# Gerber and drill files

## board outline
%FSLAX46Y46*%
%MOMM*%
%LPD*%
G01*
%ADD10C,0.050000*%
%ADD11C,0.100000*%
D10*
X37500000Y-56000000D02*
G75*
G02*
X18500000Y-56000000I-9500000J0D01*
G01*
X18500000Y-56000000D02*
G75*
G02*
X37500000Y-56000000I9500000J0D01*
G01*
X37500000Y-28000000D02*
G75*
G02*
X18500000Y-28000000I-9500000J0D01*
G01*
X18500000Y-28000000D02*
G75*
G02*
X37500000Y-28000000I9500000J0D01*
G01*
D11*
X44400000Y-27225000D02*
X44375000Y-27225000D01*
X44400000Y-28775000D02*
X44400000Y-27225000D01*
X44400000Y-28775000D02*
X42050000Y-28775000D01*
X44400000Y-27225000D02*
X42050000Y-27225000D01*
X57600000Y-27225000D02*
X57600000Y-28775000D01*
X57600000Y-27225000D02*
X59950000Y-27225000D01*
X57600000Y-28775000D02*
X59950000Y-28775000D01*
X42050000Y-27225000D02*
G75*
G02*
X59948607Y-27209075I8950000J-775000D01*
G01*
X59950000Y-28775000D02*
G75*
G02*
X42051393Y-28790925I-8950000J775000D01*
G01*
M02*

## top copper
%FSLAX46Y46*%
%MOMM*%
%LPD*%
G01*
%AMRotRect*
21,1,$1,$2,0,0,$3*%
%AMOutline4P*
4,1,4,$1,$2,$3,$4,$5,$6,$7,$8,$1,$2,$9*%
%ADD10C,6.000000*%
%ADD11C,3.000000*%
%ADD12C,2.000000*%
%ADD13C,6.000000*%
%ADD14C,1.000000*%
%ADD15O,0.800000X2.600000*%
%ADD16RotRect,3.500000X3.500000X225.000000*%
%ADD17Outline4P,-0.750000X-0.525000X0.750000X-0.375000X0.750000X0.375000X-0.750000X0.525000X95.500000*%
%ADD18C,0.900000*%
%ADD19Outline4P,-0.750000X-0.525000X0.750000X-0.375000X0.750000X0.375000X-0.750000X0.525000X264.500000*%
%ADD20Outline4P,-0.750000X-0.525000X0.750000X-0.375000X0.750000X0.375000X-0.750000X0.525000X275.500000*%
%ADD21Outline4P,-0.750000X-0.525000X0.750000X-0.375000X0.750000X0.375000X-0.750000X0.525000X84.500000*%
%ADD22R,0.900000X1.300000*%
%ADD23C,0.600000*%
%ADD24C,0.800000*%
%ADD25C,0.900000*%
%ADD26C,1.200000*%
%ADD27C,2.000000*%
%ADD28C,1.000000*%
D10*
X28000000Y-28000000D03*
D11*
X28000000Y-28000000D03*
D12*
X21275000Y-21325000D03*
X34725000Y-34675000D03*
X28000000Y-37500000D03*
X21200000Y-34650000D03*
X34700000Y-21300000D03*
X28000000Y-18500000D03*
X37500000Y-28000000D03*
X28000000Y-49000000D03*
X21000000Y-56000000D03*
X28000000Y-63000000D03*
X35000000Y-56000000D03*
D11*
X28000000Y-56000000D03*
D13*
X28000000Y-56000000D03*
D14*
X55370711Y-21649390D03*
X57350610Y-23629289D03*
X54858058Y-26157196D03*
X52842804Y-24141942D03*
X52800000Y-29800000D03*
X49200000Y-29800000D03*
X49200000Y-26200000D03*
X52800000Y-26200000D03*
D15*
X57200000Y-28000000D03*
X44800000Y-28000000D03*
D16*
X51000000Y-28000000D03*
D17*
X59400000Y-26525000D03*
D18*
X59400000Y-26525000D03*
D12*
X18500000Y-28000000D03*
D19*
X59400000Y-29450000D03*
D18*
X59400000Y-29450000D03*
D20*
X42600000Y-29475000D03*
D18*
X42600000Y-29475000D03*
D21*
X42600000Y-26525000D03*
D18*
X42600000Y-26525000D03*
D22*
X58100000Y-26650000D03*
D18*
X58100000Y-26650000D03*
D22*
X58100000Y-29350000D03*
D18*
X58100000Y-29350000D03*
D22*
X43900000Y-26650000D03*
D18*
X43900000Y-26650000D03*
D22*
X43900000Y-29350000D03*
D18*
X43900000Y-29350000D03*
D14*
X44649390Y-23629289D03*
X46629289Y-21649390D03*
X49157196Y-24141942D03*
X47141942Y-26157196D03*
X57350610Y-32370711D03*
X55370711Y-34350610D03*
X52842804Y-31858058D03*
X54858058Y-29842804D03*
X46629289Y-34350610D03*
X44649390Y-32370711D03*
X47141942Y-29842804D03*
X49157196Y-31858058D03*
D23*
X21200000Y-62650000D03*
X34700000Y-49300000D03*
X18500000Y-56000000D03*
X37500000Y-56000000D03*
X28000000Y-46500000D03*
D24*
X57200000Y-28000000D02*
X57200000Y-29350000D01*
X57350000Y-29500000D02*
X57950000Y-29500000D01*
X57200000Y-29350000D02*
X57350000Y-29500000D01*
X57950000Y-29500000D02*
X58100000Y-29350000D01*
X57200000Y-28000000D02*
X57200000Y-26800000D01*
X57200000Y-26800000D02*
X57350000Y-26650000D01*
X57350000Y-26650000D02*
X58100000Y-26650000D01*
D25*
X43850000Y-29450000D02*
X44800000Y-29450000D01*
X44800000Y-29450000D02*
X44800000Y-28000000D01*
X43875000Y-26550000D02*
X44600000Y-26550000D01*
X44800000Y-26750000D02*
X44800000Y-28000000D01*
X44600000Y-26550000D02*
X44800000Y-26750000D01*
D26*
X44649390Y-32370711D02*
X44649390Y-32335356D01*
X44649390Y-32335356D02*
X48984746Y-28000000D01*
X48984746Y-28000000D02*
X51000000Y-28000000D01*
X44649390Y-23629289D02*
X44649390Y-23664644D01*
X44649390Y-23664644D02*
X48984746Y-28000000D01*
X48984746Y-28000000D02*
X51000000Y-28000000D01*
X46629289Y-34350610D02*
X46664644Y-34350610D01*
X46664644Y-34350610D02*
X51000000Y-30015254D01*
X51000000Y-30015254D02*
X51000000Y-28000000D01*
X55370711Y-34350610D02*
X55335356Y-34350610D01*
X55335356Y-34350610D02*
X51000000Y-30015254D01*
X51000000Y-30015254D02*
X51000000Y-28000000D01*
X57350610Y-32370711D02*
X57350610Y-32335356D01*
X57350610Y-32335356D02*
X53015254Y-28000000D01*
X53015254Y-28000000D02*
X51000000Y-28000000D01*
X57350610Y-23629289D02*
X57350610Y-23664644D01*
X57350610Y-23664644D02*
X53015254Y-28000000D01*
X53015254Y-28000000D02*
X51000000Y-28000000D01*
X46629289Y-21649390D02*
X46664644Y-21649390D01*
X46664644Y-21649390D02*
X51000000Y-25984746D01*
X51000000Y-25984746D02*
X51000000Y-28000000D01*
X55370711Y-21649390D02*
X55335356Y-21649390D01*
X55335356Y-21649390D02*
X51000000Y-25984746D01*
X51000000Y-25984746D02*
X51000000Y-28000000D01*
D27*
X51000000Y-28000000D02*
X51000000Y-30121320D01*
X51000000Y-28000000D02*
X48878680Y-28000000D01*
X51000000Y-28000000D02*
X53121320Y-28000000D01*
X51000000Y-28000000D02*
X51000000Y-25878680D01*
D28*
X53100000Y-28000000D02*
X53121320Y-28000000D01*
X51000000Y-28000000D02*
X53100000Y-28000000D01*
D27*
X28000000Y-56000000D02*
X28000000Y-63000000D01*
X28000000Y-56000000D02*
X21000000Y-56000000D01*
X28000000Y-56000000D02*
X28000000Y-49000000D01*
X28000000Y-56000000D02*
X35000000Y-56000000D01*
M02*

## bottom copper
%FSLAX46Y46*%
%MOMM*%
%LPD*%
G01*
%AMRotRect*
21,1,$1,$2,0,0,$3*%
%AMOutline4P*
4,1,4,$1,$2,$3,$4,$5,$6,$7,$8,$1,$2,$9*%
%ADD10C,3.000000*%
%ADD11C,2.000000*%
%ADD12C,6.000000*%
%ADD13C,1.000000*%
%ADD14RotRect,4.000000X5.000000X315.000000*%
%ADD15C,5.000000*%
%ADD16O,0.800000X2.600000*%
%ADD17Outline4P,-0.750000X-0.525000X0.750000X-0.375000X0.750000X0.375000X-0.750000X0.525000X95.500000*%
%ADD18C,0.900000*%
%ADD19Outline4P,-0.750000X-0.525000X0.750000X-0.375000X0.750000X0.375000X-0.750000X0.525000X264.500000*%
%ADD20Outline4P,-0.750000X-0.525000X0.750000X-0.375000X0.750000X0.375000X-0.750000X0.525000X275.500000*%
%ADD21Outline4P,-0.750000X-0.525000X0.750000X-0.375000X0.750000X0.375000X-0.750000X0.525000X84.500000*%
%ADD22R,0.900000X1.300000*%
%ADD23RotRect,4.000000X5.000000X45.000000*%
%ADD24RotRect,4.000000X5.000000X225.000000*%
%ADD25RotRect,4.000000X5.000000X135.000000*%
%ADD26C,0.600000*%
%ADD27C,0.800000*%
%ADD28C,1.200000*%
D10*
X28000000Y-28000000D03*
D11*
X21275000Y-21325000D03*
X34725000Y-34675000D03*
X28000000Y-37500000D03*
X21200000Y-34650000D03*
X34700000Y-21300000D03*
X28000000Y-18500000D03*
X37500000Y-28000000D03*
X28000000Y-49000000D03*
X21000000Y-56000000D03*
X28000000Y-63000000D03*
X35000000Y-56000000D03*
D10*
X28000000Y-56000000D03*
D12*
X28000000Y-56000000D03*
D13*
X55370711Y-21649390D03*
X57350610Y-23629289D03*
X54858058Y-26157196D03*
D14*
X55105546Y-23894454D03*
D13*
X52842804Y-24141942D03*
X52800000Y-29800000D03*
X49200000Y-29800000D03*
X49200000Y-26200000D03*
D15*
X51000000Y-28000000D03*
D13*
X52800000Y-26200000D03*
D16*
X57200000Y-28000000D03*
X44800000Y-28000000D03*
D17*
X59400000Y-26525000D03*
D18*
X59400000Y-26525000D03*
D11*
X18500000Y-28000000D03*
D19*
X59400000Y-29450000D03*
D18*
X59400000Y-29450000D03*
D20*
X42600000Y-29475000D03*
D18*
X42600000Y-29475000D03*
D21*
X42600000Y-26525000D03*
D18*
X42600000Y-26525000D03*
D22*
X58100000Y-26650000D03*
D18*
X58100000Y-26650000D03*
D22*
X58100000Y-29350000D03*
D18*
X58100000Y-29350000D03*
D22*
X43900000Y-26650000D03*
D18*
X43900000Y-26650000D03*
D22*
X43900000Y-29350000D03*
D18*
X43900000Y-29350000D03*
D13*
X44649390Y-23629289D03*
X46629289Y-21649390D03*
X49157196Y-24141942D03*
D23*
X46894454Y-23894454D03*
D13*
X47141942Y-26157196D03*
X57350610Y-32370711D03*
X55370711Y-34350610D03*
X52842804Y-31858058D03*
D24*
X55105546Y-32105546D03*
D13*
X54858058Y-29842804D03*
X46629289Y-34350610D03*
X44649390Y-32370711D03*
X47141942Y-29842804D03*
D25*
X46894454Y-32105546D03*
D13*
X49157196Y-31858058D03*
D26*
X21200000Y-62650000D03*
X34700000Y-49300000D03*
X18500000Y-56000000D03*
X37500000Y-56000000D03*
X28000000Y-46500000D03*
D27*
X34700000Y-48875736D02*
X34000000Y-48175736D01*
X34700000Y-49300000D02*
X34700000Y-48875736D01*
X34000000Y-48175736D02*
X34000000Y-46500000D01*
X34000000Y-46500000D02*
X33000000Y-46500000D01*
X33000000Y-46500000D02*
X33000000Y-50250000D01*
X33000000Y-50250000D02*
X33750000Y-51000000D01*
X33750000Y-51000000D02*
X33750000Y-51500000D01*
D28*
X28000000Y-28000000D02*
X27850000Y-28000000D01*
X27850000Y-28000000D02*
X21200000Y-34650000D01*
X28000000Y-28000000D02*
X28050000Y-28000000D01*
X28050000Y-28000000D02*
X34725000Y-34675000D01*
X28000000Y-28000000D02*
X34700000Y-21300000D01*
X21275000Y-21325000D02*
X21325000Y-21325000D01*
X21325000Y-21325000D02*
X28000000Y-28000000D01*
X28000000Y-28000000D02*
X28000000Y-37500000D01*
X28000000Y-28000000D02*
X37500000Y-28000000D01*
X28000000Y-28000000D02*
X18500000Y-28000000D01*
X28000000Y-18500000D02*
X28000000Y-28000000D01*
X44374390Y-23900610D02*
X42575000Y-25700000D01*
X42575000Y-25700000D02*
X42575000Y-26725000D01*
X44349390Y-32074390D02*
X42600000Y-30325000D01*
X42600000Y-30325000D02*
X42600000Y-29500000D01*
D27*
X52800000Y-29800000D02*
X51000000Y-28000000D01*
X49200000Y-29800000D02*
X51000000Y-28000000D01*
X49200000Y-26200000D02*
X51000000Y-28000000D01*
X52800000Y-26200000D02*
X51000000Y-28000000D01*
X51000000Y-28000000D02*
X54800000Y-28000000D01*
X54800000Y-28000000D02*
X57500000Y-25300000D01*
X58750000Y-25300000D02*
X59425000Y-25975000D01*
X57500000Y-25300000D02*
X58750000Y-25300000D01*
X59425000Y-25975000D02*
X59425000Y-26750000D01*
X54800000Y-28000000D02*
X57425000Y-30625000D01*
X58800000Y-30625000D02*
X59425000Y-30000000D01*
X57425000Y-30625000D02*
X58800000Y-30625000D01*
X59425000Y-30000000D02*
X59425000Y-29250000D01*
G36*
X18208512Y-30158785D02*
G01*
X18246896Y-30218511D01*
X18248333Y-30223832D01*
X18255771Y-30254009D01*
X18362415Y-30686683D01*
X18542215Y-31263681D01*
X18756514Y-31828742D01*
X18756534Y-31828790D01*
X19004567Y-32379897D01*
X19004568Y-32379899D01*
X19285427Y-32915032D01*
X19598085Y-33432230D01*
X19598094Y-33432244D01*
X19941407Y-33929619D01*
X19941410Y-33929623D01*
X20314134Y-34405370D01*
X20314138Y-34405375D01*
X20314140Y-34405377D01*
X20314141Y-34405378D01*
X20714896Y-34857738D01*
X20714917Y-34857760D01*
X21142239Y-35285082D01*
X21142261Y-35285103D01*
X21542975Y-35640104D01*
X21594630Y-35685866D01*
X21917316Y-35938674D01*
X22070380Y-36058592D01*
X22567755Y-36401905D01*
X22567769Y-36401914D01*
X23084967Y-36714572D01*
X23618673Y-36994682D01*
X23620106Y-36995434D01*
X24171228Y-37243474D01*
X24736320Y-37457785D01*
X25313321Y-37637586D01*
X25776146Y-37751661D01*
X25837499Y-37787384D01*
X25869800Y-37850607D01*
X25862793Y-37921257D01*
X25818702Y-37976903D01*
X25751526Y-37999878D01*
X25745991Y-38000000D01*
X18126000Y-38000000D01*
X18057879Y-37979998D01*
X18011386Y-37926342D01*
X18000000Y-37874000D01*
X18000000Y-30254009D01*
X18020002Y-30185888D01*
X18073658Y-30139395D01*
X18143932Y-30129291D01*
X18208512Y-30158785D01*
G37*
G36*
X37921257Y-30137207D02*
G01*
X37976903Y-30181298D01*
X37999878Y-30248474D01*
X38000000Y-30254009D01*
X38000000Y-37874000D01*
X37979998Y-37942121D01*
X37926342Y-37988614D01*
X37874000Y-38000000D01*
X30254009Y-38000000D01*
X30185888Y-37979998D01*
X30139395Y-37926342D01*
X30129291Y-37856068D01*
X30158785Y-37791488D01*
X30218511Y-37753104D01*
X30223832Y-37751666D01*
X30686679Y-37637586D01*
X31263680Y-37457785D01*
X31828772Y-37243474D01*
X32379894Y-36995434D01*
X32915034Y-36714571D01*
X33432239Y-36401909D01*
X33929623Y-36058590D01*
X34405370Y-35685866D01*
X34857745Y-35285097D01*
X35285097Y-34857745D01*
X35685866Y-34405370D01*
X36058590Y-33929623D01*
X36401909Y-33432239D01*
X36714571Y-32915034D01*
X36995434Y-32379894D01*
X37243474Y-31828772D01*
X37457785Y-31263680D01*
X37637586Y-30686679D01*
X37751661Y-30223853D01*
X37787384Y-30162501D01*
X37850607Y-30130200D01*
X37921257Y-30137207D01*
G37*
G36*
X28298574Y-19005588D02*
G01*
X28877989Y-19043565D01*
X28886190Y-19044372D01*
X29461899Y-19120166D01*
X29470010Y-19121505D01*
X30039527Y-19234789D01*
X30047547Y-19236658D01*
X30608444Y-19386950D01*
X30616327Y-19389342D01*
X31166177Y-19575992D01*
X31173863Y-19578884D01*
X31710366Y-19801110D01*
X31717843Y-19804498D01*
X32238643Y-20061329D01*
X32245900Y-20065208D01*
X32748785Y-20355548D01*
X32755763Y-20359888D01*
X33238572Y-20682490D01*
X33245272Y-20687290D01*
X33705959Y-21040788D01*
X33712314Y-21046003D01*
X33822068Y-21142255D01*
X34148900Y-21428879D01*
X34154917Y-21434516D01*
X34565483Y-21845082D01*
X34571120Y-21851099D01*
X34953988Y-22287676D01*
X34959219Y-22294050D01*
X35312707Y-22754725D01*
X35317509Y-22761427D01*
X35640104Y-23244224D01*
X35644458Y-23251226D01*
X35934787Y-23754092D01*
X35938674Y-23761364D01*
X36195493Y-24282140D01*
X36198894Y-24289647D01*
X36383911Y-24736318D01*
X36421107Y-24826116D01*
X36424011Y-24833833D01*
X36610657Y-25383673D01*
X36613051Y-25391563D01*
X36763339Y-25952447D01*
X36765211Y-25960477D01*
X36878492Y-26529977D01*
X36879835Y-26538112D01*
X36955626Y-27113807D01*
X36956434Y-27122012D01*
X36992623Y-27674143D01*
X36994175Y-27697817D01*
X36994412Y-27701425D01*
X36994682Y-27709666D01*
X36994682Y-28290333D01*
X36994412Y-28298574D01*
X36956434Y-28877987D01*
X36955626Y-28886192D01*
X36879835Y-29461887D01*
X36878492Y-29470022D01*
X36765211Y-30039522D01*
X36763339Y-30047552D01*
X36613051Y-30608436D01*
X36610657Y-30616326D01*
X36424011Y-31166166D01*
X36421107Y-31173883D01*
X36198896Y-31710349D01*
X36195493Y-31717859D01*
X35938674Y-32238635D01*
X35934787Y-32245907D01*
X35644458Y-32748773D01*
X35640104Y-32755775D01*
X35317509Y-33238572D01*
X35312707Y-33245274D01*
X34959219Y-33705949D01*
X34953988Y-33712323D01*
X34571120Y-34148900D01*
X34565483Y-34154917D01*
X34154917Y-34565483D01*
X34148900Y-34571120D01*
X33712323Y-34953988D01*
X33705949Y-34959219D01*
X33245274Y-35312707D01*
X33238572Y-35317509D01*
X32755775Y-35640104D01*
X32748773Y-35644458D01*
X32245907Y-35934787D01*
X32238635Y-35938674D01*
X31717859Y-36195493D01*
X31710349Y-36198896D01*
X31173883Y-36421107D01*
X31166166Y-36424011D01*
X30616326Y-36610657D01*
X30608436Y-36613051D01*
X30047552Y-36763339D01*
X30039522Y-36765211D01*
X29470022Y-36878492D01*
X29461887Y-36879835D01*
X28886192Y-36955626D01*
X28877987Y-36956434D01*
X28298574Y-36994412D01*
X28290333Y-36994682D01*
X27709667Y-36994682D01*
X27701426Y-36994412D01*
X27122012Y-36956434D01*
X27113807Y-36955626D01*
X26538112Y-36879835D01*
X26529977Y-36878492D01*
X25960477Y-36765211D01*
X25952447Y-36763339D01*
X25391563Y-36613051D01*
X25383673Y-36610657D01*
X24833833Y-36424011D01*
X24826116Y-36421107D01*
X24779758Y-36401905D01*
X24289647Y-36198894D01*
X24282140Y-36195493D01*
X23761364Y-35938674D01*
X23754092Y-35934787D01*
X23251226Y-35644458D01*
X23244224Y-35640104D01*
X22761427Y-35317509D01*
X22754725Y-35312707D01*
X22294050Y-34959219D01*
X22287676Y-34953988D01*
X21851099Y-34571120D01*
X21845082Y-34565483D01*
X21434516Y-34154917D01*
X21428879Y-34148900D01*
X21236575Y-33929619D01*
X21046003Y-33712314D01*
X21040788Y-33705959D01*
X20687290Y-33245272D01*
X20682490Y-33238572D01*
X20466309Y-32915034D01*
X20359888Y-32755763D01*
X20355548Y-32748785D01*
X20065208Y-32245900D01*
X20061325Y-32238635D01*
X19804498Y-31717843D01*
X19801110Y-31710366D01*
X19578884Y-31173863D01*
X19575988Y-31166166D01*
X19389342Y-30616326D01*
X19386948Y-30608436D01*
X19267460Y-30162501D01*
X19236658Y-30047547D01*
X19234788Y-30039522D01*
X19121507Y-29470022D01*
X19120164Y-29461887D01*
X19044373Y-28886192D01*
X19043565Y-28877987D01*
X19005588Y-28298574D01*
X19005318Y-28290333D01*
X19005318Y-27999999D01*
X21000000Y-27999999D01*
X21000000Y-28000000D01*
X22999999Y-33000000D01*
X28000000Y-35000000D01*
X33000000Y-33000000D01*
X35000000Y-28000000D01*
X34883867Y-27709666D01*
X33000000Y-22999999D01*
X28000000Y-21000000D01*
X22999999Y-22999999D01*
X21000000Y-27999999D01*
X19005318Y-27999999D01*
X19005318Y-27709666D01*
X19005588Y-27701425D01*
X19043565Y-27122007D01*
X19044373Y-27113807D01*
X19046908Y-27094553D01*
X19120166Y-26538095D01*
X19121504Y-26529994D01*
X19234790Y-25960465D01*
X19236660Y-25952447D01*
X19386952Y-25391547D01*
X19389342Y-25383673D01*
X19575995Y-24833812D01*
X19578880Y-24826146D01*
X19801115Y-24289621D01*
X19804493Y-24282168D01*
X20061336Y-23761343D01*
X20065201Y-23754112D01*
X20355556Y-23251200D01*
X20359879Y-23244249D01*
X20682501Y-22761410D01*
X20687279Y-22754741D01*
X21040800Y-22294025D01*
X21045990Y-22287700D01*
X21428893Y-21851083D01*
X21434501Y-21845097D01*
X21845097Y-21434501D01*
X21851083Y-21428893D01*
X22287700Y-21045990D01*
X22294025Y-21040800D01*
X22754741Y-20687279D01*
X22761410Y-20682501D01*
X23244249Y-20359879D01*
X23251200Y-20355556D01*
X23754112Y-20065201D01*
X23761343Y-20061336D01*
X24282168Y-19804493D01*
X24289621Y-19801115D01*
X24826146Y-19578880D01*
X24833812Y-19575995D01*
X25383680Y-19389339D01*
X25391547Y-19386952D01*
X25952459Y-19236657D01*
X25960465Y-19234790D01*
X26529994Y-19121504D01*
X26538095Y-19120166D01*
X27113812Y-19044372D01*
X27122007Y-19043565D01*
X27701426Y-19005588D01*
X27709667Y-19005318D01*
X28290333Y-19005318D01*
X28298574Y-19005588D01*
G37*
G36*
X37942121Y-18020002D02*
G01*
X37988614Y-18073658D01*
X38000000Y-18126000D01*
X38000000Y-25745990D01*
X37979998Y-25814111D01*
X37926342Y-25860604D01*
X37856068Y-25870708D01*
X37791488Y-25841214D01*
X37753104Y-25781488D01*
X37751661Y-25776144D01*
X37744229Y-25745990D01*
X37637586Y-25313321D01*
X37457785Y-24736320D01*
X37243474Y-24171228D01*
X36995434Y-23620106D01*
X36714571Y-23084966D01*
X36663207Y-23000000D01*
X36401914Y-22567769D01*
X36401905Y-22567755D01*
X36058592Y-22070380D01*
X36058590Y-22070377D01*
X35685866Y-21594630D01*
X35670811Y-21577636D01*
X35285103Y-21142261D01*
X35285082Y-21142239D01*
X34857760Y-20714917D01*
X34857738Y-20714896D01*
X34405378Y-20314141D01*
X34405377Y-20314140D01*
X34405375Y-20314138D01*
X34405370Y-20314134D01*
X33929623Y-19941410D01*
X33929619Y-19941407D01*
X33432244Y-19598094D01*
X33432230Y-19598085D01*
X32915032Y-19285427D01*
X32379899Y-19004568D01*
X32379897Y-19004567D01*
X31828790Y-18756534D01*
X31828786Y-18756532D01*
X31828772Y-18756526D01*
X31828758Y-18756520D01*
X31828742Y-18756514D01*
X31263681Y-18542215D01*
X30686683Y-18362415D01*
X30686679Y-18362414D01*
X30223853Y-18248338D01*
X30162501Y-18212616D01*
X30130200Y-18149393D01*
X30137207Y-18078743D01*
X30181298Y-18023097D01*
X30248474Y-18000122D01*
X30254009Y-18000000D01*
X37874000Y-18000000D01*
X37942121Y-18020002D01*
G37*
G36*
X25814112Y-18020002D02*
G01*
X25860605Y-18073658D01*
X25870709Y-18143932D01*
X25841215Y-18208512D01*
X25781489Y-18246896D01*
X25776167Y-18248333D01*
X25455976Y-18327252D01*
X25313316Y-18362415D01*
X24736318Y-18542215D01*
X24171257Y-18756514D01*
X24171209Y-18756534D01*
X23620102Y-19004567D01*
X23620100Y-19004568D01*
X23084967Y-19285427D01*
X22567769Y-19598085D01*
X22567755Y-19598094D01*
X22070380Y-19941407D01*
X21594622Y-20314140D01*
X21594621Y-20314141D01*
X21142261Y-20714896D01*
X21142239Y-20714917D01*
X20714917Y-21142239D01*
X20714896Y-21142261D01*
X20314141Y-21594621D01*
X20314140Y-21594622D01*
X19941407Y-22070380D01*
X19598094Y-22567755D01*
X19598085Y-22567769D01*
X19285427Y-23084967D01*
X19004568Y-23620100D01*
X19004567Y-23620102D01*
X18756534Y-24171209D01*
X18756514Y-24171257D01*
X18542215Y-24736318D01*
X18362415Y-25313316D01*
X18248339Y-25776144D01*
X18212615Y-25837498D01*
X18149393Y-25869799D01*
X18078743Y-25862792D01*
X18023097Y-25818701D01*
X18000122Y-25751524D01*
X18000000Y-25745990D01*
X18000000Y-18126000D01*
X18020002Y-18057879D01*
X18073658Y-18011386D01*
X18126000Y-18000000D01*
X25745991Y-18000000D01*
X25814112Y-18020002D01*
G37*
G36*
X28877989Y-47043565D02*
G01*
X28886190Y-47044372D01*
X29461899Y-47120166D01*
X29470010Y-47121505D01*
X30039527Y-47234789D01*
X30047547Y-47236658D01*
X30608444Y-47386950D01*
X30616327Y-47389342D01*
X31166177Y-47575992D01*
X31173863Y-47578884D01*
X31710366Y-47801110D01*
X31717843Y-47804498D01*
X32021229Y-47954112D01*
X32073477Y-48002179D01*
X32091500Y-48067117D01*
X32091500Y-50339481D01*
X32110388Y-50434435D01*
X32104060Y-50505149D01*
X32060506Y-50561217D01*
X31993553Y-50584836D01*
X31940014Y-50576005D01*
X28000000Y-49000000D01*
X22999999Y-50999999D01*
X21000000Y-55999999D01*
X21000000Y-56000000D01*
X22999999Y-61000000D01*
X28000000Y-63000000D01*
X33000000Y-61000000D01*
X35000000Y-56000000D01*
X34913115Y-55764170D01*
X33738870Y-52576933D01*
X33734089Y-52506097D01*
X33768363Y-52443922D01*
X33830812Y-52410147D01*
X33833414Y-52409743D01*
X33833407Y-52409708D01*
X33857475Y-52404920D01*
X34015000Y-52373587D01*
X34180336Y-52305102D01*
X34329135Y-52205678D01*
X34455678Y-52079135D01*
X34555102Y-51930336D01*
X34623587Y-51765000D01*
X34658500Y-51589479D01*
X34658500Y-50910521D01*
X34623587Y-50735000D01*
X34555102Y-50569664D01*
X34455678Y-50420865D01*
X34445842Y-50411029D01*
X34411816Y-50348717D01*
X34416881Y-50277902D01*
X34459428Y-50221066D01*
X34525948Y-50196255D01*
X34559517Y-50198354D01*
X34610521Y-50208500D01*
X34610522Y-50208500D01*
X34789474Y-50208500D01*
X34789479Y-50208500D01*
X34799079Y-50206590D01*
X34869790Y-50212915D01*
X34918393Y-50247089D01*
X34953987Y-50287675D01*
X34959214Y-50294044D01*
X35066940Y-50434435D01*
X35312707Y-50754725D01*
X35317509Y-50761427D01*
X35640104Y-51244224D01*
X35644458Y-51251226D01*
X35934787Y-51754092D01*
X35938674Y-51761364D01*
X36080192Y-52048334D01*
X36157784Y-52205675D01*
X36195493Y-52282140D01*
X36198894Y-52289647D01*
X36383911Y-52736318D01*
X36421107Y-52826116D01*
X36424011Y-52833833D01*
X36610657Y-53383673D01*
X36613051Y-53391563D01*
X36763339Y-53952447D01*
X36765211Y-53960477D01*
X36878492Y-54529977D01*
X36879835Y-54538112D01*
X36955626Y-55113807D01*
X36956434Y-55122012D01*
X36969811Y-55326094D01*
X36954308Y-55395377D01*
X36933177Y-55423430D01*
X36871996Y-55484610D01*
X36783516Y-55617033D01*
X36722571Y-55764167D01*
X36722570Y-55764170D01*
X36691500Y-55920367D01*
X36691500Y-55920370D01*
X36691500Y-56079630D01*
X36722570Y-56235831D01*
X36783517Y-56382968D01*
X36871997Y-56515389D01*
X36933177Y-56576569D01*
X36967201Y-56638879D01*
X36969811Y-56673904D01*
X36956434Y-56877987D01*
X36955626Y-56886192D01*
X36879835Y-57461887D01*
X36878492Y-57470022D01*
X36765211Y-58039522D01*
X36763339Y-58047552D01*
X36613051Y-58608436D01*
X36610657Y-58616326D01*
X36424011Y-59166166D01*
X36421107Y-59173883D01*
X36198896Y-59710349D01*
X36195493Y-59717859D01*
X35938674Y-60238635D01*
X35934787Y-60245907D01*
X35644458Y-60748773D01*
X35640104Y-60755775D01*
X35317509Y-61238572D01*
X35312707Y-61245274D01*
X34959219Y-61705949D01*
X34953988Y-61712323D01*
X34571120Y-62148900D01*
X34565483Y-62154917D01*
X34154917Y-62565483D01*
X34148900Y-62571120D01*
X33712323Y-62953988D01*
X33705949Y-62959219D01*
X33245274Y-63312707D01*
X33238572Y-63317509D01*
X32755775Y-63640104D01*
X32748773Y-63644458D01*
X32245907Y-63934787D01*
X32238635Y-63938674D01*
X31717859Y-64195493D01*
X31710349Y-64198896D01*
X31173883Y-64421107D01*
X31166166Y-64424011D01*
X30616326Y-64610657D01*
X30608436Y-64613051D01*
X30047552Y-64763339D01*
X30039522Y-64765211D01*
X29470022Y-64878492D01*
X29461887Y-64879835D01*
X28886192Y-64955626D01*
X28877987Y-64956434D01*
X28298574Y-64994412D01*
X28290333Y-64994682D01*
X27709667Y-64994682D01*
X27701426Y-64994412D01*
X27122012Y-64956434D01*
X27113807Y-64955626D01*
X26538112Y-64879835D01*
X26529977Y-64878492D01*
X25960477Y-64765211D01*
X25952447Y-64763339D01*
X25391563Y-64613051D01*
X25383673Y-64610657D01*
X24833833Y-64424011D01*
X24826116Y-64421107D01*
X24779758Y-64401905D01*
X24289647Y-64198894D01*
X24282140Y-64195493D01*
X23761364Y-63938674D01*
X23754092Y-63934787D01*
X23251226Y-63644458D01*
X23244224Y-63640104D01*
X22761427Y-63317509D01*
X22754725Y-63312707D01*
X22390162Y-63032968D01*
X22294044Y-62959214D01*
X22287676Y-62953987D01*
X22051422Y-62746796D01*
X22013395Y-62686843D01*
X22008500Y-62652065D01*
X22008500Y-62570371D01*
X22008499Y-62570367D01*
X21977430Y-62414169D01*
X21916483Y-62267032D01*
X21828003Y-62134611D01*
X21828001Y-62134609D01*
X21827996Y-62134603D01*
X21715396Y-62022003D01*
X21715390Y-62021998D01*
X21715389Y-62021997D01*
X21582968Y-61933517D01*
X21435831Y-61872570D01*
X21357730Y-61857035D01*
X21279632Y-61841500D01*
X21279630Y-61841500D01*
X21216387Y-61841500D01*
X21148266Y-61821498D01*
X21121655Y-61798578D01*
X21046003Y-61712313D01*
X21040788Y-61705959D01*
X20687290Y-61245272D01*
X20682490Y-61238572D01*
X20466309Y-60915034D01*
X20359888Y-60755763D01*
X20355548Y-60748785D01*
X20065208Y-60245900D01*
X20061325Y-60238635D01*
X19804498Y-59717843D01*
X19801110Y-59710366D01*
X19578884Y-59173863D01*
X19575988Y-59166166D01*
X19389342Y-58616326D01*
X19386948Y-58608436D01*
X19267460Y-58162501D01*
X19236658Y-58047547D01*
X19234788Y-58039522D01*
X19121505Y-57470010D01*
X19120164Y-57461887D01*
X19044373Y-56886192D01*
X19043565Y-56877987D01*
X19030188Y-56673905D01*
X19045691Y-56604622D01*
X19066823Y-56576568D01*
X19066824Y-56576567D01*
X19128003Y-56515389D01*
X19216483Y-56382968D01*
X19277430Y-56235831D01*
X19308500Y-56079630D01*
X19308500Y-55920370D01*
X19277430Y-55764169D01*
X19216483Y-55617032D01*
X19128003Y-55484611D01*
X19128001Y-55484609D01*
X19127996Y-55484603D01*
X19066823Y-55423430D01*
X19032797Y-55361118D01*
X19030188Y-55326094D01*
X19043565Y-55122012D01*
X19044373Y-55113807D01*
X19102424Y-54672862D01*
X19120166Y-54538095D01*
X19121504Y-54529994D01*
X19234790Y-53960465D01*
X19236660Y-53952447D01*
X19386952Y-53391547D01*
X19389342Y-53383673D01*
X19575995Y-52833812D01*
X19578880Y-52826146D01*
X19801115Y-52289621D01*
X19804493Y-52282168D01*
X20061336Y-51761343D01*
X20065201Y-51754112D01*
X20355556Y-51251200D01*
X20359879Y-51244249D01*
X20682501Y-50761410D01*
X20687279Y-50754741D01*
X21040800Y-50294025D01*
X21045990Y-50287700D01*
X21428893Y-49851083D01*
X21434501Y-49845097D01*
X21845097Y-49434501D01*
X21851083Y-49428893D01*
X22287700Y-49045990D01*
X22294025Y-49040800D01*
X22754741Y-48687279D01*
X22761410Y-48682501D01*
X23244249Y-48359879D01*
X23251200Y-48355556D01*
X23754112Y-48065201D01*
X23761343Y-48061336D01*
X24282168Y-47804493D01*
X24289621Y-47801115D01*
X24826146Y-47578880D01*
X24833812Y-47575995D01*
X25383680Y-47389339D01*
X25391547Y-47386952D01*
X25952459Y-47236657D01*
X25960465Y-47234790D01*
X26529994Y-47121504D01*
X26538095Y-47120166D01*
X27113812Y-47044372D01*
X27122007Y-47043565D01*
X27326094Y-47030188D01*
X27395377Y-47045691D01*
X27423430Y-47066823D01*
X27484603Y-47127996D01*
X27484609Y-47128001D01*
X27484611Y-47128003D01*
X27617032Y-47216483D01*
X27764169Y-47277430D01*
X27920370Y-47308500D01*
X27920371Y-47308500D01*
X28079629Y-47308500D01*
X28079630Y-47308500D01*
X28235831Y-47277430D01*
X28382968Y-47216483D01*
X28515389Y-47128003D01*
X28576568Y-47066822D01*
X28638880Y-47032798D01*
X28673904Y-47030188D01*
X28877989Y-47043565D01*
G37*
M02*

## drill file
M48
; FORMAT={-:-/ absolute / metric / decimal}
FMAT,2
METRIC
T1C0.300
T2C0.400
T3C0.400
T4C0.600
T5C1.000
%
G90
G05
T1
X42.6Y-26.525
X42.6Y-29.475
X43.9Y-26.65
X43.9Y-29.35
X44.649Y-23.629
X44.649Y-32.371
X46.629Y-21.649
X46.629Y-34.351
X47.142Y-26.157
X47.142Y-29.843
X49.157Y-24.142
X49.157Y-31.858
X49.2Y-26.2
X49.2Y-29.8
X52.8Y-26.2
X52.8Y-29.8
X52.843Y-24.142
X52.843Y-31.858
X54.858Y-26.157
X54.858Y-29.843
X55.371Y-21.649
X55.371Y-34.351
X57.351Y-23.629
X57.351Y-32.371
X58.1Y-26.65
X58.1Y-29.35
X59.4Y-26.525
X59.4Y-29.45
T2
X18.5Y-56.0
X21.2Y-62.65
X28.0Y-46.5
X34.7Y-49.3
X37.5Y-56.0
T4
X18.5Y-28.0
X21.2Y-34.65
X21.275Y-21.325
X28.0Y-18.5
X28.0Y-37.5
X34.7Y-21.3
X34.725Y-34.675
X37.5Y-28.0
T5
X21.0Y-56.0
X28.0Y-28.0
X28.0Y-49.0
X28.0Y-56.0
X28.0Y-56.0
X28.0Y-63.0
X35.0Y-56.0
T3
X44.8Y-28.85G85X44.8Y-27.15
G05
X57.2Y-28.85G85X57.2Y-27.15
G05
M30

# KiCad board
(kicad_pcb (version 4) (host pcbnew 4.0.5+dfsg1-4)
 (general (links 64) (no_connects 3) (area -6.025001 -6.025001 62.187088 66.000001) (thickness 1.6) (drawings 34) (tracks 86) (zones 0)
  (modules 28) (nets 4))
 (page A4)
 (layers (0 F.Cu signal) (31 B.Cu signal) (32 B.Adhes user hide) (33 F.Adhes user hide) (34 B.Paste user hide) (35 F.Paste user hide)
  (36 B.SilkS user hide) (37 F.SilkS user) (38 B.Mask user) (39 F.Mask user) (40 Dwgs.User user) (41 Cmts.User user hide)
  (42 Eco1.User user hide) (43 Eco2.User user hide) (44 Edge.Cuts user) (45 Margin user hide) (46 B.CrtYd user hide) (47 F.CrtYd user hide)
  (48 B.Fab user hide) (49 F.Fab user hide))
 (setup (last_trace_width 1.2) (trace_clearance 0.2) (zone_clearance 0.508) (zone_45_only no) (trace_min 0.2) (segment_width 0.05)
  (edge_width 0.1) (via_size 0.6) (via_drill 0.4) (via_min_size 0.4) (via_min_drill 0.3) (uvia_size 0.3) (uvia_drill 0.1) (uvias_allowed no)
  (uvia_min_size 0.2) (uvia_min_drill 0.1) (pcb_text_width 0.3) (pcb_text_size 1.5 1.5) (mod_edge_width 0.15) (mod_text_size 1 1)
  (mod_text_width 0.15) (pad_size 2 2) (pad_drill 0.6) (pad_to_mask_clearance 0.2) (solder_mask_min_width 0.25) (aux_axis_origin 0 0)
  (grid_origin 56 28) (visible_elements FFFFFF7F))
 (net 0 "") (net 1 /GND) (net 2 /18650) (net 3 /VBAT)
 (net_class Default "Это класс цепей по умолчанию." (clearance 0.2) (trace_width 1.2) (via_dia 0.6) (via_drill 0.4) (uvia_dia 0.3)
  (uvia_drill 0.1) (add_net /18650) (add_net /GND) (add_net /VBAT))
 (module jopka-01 (layer F.Cu) (at 28 28)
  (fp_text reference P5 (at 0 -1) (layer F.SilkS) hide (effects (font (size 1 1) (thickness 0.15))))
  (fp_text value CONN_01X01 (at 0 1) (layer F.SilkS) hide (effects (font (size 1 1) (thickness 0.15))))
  (pad 1 smd circle (at 0 0) (size 6 6) (layers F.Cu F.Paste F.Mask) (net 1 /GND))
  (pad 2 thru_hole circle (at 0 0) (size 3 3) (drill 1) (layers *.Mask B.Cu) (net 1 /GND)))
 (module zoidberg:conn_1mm (layer F.Cu) (at 21.275 21.325)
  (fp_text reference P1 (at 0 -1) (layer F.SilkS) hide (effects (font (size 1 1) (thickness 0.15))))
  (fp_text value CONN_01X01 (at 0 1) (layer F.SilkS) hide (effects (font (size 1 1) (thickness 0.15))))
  (pad 1 thru_hole circle (at 0 0) (size 2 2) (drill 0.6) (layers *.Cu) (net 1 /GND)))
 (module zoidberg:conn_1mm (layer F.Cu) (at 34.725 34.675)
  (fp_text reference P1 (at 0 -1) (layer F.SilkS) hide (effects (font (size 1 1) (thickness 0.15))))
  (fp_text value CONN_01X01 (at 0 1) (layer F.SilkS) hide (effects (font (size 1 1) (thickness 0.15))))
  (pad 1 thru_hole circle (at 0 0) (size 2 2) (drill 0.6) (layers *.Cu) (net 1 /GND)))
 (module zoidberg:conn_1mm (layer F.Cu) (at 28 37.5)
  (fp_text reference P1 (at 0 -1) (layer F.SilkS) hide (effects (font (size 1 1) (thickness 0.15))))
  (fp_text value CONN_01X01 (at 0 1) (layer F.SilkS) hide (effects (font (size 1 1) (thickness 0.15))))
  (pad 1 thru_hole circle (at 0 0) (size 2 2) (drill 0.6) (layers *.Cu) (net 1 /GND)))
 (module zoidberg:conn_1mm (layer F.Cu) (at 21.2 34.65)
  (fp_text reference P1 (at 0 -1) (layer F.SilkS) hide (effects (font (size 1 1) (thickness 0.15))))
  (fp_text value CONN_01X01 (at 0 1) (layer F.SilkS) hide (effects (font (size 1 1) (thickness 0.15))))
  (pad 1 thru_hole circle (at 0 0) (size 2 2) (drill 0.6) (layers *.Cu) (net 1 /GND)))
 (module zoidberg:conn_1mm (layer F.Cu) (at 34.7 21.3)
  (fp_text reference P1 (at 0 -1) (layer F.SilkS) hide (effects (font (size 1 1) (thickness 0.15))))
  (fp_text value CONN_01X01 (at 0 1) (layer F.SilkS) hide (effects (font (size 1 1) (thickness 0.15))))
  (pad 1 thru_hole circle (at 0 0) (size 2 2) (drill 0.6) (layers *.Cu) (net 1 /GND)))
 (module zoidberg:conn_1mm (layer F.Cu) (at 28 18.5)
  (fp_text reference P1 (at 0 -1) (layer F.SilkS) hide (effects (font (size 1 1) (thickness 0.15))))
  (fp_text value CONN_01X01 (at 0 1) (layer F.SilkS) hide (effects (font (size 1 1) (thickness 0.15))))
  (pad 1 thru_hole circle (at 0 0) (size 2 2) (drill 0.6) (layers *.Cu) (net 1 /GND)))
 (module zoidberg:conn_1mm (layer F.Cu) (at 37.5 28)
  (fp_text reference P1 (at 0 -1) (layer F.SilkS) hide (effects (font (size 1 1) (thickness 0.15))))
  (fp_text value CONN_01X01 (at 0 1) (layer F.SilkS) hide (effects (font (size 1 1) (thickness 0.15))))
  (pad 1 thru_hole circle (at 0 0) (size 2 2) (drill 0.6) (layers *.Cu) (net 1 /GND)))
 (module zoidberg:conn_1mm (layer F.Cu) (at 28 49)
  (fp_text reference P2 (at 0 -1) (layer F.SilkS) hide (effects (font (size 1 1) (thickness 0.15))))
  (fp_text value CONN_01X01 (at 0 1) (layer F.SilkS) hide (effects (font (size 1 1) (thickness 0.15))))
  (pad 1 thru_hole circle (at 0 0) (size 2 2) (drill 1) (layers *.Cu) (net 1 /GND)))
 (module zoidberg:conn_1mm (layer F.Cu) (at 21 56)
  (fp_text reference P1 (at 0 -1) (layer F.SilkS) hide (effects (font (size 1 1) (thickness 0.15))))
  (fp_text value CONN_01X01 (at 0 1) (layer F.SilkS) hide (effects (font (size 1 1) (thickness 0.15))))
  (pad 1 thru_hole circle (at 0 0) (size 2 2) (drill 1) (layers *.Cu) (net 1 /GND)))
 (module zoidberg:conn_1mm (layer F.Cu) (at 28 63)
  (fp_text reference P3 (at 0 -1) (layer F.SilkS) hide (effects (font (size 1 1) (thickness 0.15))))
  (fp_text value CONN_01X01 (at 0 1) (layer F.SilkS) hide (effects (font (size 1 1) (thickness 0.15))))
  (pad 1 thru_hole circle (at 0 0) (size 2 2) (drill 1) (layers *.Cu) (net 1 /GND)))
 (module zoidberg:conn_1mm (layer F.Cu) (at 35 56)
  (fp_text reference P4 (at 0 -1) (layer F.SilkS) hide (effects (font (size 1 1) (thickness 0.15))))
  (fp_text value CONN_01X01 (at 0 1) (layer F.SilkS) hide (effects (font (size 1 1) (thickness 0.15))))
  (pad 1 thru_hole circle (at 0 0) (size 2 2) (drill 1) (layers *.Cu) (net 1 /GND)))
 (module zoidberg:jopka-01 (layer F.Cu) (at 28 56)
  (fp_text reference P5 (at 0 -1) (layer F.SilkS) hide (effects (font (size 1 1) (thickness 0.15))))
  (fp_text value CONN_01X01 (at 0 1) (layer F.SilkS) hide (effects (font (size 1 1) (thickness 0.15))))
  (pad 2 thru_hole circle (at 0 0) (size 3 3) (drill 1) (layers *.Mask B.Cu))
  (pad 1 thru_hole circle (at 0 0) (size 6 6) (drill 1) (layers *.Cu *.Mask) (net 1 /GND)))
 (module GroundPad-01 (layer F.Cu) (at 55.3 23.7 315)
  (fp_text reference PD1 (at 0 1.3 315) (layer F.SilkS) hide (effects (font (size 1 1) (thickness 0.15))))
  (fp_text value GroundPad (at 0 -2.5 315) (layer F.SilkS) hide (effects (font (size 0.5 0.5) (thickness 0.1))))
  (pad 2 thru_hole circle (at -1.4 -1.5 315) (size 1 1) (drill 0.3) (layers *.Cu) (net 1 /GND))
  (pad 3 thru_hole circle (at 1.4 -1.5 315) (size 1 1) (drill 0.3) (layers *.Cu) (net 1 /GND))
  (pad 5 thru_hole circle (at 1.425 2.05 315) (size 1 1) (drill 0.3) (layers *.Cu) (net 1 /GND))
  (pad 1 smd rect (at 0 0.274999 315) (size 4 5) (layers B.Cu B.Paste B.Mask) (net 1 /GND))
  (pad 4 thru_hole circle (at -1.425 2.05 315) (size 1 1) (drill 0.3) (layers *.Cu) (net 1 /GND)))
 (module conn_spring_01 (layer B.Cu) (at 51 28 270)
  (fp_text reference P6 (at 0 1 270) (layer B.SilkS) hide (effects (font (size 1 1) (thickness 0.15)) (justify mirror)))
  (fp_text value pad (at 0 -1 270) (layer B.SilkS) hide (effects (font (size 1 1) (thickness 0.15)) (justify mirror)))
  (pad 4 thru_hole circle (at 1.8 -1.8 270) (size 1 1) (drill 0.3) (layers *.Cu) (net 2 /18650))
  (pad 3 thru_hole circle (at 1.8 1.8 270) (size 1 1) (drill 0.3) (layers *.Cu) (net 2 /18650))
  (pad 2 thru_hole circle (at -1.8 1.8 270) (size 1 1) (drill 0.3) (layers *.Cu) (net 2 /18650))
  (pad 1 smd circle (at 0 0 270) (size 5 5) (layers B.Cu B.Paste B.Mask) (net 2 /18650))
  (pad 5 thru_hole circle (at -1.8 -1.8 270) (size 1 1) (drill 0.3) (layers *.Cu) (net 2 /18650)))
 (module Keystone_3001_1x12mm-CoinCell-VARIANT (layer F.Cu) (at 51 28 180)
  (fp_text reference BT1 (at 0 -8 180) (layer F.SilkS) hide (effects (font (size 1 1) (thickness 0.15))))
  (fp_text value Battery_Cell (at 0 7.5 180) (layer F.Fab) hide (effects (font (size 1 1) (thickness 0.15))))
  (pad 1 thru_hole oval (at -6.2 0 180) (size 0.8 2.6) (drill oval 0.4 2.1) (layers *.Cu *.Mask) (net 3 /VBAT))
  (pad 1 thru_hole oval (at 6.2 0 180) (size 0.8 2.6) (drill oval 0.4 2.1) (layers *.Cu *.Mask) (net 3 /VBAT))
  (pad 2 smd rect (at 0 0 225) (size 3.5 3.5) (layers F.Cu F.Mask) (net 1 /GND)))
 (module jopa (layer F.Cu) (at 59.4 26.525 95.5)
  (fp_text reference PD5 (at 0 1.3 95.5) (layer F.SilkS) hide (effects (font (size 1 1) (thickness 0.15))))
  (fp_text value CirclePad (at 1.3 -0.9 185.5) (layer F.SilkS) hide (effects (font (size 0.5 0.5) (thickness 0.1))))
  (pad 1 smd trapezoid (at 0 0 95.5) (size 1.5 0.9) (rect_delta 0.15 0) (layers F.Cu F.Paste F.Mask) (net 2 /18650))
  (pad 2 smd trapezoid (at 0 0 95.5) (size 1.5 0.9) (rect_delta 0.15 0) (layers B.Cu F.Paste B.Mask) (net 2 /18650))
  (pad 3 thru_hole circle (at 0 0 95.5) (size 0.9 0.9) (drill 0.3) (layers *.Cu *.Mask) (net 2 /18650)))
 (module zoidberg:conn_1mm (layer F.Cu) (at 18.5 28)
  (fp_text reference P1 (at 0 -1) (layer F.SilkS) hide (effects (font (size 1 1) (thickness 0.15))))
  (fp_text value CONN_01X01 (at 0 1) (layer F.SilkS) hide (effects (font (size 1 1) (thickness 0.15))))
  (pad 1 thru_hole circle (at 0 0) (size 2 2) (drill 0.6) (layers *.Cu) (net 1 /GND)))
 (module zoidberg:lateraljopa (layer F.Cu) (at 59.4 29.45 264.5)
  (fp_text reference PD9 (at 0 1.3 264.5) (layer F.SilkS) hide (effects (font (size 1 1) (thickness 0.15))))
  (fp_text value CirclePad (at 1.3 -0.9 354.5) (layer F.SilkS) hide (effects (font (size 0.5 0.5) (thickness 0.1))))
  (pad 1 smd trapezoid (at 0 0 264.5) (size 1.5 0.9) (rect_delta 0.15 0) (layers F.Cu F.Paste F.Mask) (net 2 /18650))
  (pad 2 smd trapezoid (at 0 0 264.5) (size 1.5 0.9) (rect_delta 0.15 0) (layers B.Cu F.Paste B.Mask) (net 2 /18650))
  (pad 3 thru_hole circle (at 0 0 264.5) (size 0.9 0.9) (drill 0.3) (layers *.Cu *.Mask) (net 2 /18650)))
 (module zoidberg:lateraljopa (layer F.Cu) (at 42.6 29.475 275.5)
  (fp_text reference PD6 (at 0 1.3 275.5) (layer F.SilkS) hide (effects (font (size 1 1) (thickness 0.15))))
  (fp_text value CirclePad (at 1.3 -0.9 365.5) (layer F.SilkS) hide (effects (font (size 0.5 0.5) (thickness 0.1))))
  (pad 1 smd trapezoid (at 0 0 275.5) (size 1.5 0.9) (rect_delta 0.15 0) (layers F.Cu F.Paste F.Mask) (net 1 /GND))
  (pad 2 smd trapezoid (at 0 0 275.5) (size 1.5 0.9) (rect_delta 0.15 0) (layers B.Cu F.Paste B.Mask) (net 1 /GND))
  (pad 3 thru_hole circle (at 0 0 275.5) (size 0.9 0.9) (drill 0.3) (layers *.Cu *.Mask) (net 1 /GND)))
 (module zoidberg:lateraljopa (layer F.Cu) (at 42.6 26.525 84.5)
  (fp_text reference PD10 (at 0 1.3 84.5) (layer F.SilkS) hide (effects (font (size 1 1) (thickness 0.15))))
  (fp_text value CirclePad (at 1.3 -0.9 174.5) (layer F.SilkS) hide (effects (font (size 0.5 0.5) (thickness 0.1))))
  (pad 1 smd trapezoid (at 0 0 84.5) (size 1.5 0.9) (rect_delta 0.15 0) (layers F.Cu F.Paste F.Mask) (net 1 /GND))
  (pad 2 smd trapezoid (at 0 0 84.5) (size 1.5 0.9) (rect_delta 0.15 0) (layers B.Cu F.Paste B.Mask) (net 1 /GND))
  (pad 3 thru_hole circle (at 0 0 84.5) (size 0.9 0.9) (drill 0.3) (layers *.Cu *.Mask) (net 1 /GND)))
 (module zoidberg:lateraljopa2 (layer F.Cu) (at 58.1 26.65 90)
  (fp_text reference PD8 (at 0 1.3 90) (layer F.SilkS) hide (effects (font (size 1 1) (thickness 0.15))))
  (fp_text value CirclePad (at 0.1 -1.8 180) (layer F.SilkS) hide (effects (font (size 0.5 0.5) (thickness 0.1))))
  (pad 1 smd rect (at 0 0 90) (size 1.3 0.9) (layers F.Cu F.Paste F.Mask) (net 3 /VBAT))
  (pad 2 smd rect (at 0 0 90) (size 1.3 0.9) (layers B.Cu F.Paste B.Mask) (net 3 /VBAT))
  (pad 3 thru_hole circle (at 0 0 90) (size 0.9 0.9) (drill 0.3) (layers *.Cu *.Mask) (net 3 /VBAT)))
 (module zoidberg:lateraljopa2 (layer F.Cu) (at 58.1 29.35 90)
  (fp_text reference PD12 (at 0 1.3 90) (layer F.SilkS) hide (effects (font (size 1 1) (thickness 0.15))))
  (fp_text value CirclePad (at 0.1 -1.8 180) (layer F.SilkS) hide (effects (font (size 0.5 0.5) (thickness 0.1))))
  (pad 1 smd rect (at 0 0 90) (size 1.3 0.9) (layers F.Cu F.Paste F.Mask) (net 3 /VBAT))
  (pad 2 smd rect (at 0 0 90) (size 1.3 0.9) (layers B.Cu F.Paste B.Mask) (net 3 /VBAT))
  (pad 3 thru_hole circle (at 0 0 90) (size 0.9 0.9) (drill 0.3) (layers *.Cu *.Mask) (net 3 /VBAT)))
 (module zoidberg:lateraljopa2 (layer F.Cu) (at 43.9 26.65 90)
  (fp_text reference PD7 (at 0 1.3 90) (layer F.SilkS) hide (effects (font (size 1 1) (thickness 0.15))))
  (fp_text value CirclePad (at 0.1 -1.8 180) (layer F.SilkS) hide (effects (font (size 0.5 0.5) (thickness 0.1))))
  (pad 1 smd rect (at 0 0 90) (size 1.3 0.9) (layers F.Cu F.Paste F.Mask) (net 3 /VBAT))
  (pad 2 smd rect (at 0 0 90) (size 1.3 0.9) (layers B.Cu F.Paste B.Mask) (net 3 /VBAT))
  (pad 3 thru_hole circle (at 0 0 90) (size 0.9 0.9) (drill 0.3) (layers *.Cu *.Mask) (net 3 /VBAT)))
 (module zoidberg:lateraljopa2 (layer F.Cu) (at 43.9 29.35 90)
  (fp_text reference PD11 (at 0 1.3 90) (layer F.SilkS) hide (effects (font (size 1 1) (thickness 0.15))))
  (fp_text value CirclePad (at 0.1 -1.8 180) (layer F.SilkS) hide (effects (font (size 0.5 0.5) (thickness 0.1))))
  (pad 1 smd rect (at 0 0 90) (size 1.3 0.9) (layers F.Cu F.Paste F.Mask) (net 3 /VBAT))
  (pad 2 smd rect (at 0 0 90) (size 1.3 0.9) (layers B.Cu F.Paste B.Mask) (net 3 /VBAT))
  (pad 3 thru_hole circle (at 0 0 90) (size 0.9 0.9) (drill 0.3) (layers *.Cu *.Mask) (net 3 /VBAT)))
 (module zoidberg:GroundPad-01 (layer F.Cu) (at 46.7 23.7 45)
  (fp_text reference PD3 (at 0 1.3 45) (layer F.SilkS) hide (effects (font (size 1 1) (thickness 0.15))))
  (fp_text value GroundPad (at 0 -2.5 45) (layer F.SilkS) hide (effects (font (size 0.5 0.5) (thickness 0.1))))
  (pad 2 thru_hole circle (at -1.4 -1.5 45) (size 1 1) (drill 0.3) (layers *.Cu) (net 1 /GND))
  (pad 3 thru_hole circle (at 1.4 -1.5 45) (size 1 1) (drill 0.3) (layers *.Cu) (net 1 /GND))
  (pad 5 thru_hole circle (at 1.425 2.05 45) (size 1 1) (drill 0.3) (layers *.Cu) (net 1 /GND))
  (pad 1 smd rect (at 0 0.274999 45) (size 4 5) (layers B.Cu B.Paste B.Mask) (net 1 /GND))
  (pad 4 thru_hole circle (at -1.425 2.05 45) (size 1 1) (drill 0.3) (layers *.Cu) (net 1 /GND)))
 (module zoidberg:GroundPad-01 (layer F.Cu) (at 55.3 32.3 225)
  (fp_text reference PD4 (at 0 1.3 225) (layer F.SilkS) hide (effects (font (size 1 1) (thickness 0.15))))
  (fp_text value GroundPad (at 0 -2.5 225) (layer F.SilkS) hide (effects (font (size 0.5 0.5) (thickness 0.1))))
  (pad 2 thru_hole circle (at -1.4 -1.5 225) (size 1 1) (drill 0.3) (layers *.Cu) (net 1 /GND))
  (pad 3 thru_hole circle (at 1.4 -1.5 225) (size 1 1) (drill 0.3) (layers *.Cu) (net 1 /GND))
  (pad 5 thru_hole circle (at 1.425 2.05 225) (size 1 1) (drill 0.3) (layers *.Cu) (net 1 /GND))
  (pad 1 smd rect (at 0 0.274999 225) (size 4 5) (layers B.Cu B.Paste B.Mask) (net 1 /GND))
  (pad 4 thru_hole circle (at -1.425 2.05 225) (size 1 1) (drill 0.3) (layers *.Cu) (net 1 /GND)))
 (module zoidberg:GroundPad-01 (layer F.Cu) (at 46.7 32.3 135)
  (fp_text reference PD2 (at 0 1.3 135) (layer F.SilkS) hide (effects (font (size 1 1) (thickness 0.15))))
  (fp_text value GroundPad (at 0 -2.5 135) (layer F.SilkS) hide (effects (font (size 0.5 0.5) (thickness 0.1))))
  (pad 2 thru_hole circle (at -1.4 -1.5 135) (size 1 1) (drill 0.3) (layers *.Cu) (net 1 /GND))
  (pad 3 thru_hole circle (at 1.4 -1.5 135) (size 1 1) (drill 0.3) (layers *.Cu) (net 1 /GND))
  (pad 5 thru_hole circle (at 1.425 2.05 135) (size 1 1) (drill 0.3) (layers *.Cu) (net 1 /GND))
  (pad 1 smd rect (at 0 0.274999 135) (size 4 5) (layers B.Cu B.Paste B.Mask) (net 1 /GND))
  (pad 4 thru_hole circle (at -1.425 2.05 135) (size 1 1) (drill 0.3) (layers *.Cu) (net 1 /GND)))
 (gr_circle (center 28 56) (end 37.5 56) (layer Edge.Cuts) (width 0.05))
 (gr_circle (center 28 28) (end 37.5 28) (layer Edge.Cuts) (width 0.05))
 (gr_line (start 44.4 27.225) (end 44.375 27.225) (angle 90) (layer Edge.Cuts) (width 0.1))
 (gr_line (start 44.4 28.775) (end 44.4 27.225) (angle 90) (layer Edge.Cuts) (width 0.1))
 (gr_line (start 44.4 28.775) (end 42.05 28.775) (angle 90) (layer Edge.Cuts) (width 0.1))
 (gr_line (start 44.4 27.225) (end 42.05 27.225) (angle 90) (layer Edge.Cuts) (width 0.1))
 (gr_line (start 57.6 27.225) (end 57.6 28.775) (angle 90) (layer Edge.Cuts) (width 0.1))
 (gr_line (start 57.6 27.225) (end 59.95 27.225) (angle 90) (layer Edge.Cuts) (width 0.1))
 (gr_line (start 57.6 28.775) (end 59.95 28.775) (angle 90) (layer Edge.Cuts) (width 0.1))
 (gr_arc (start 51 28) (end 42.05 27.225) (angle 170) (layer Edge.Cuts) (width 0.1))
 (gr_arc (start 51 28) (end 59.95 28.775) (angle 170) (layer Edge.Cuts) (width 0.1))
 (via (at 21.2 62.65) (size 0.6) (drill 0.4) (layers F.Cu B.Cu) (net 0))
 (via (at 34.7 49.3) (size 0.6) (drill 0.4) (layers F.Cu B.Cu) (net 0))
 (via (at 18.5 56) (size 0.6) (drill 0.4) (layers F.Cu B.Cu) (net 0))
 (via (at 37.5 56) (size 0.6) (drill 0.4) (layers F.Cu B.Cu) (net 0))
 (via (at 28 46.5) (size 0.6) (drill 0.4) (layers F.Cu B.Cu) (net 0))
 (segment (start 34.7 48.875736) (end 34 48.175736) (width 0.8) (layer B.Cu) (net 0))
 (segment (start 34.7 49.3) (end 34.7 48.875736) (width 0.8) (layer B.Cu) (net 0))
 (segment (start 34 48.175736) (end 34 46.5) (width 0.8) (layer B.Cu) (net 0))
 (segment (start 34 46.5) (end 33 46.5) (width 0.8) (layer B.Cu) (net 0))
 (segment (start 33 46.5) (end 33 50.25) (width 0.8) (layer B.Cu) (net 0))
 (segment (start 33 50.25) (end 33.75 51) (width 0.8) (layer B.Cu) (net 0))
 (segment (start 33.75 51) (end 33.75 51.5) (width 0.8) (layer B.Cu) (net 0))
 (segment (start 57.2 28) (end 57.2 29.35) (width 0.8) (layer F.Cu) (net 3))
 (segment (start 57.35 29.5) (end 57.95 29.5) (width 0.8) (layer F.Cu) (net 3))
 (segment (start 57.2 29.35) (end 57.35 29.5) (width 0.8) (layer F.Cu) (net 3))
 (segment (start 57.95 29.5) (end 58.1 29.35) (width 0.8) (layer F.Cu) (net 3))
 (segment (start 57.2 28) (end 57.2 26.8) (width 0.8) (layer F.Cu) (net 3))
 (segment (start 57.2 26.8) (end 57.35 26.65) (width 0.8) (layer F.Cu) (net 3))
 (segment (start 57.35 26.65) (end 58.1 26.65) (width 0.8) (layer F.Cu) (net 3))
 (segment (start 43.85 29.45) (end 44.8 29.45) (width 0.9) (layer F.Cu) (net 3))
 (segment (start 44.8 29.45) (end 44.8 28) (width 0.9) (layer F.Cu) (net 3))
 (segment (start 43.875 26.55) (end 44.6 26.55) (width 0.9) (layer F.Cu) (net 3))
 (segment (start 44.8 26.75) (end 44.8 28) (width 0.9) (layer F.Cu) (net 3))
 (segment (start 44.6 26.55) (end 44.8 26.75) (width 0.9) (layer F.Cu) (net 3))
 (segment (start 28 28) (end 27.85 28) (width 1.2) (layer B.Cu) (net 1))
 (segment (start 27.85 28) (end 21.2 34.65) (width 1.2) (layer B.Cu) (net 1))
 (segment (start 28 28) (end 28.05 28) (width 1.2) (layer B.Cu) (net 1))
 (segment (start 28.05 28) (end 34.725 34.675) (width 1.2) (layer B.Cu) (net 1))
 (segment (start 28 28) (end 34.7 21.3) (width 1.2) (layer B.Cu) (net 1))
 (segment (start 21.275 21.325) (end 21.325 21.325) (width 1.2) (layer B.Cu) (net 1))
 (segment (start 21.325 21.325) (end 28 28) (width 1.2) (layer B.Cu) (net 1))
 (segment (start 28 28) (end 28 37.5) (width 1.2) (layer B.Cu) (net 1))
 (segment (start 28 28) (end 37.5 28) (width 1.2) (layer B.Cu) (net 1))
 (segment (start 28 28) (end 18.5 28) (width 1.2) (layer B.Cu) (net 1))
 (segment (start 28 18.5) (end 28 28) (width 1.2) (layer B.Cu) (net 1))
 (segment (start 44.64939 32.370711) (end 44.64939 32.335356) (width 1.2) (layer F.Cu) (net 1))
 (segment (start 44.64939 32.335356) (end 48.984746 28) (width 1.2) (layer F.Cu) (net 1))
 (segment (start 48.984746 28) (end 51 28) (width 1.2) (layer F.Cu) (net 1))
 (segment (start 44.64939 23.629289) (end 44.64939 23.664644) (width 1.2) (layer F.Cu) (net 1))
 (segment (start 44.64939 23.664644) (end 48.984746 28) (width 1.2) (layer F.Cu) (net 1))
 (segment (start 48.984746 28) (end 51 28) (width 1.2) (layer F.Cu) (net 1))
 (segment (start 46.629289 34.35061) (end 46.664644 34.35061) (width 1.2) (layer F.Cu) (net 1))
 (segment (start 46.664644 34.35061) (end 51 30.015254) (width 1.2) (layer F.Cu) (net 1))
 (segment (start 51 30.015254) (end 51 28) (width 1.2) (layer F.Cu) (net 1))
 (segment (start 55.370711 34.35061) (end 55.335356 34.35061) (width 1.2) (layer F.Cu) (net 1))
 (segment (start 55.335356 34.35061) (end 51 30.015254) (width 1.2) (layer F.Cu) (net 1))
 (segment (start 51 30.015254) (end 51 28) (width 1.2) (layer F.Cu) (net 1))
 (segment (start 57.35061 32.370711) (end 57.35061 32.335356) (width 1.2) (layer F.Cu) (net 1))
 (segment (start 57.35061 32.335356) (end 53.015254 28) (width 1.2) (layer F.Cu) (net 1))
 (segment (start 53.015254 28) (end 51 28) (width 1.2) (layer F.Cu) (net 1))
 (segment (start 57.35061 23.629289) (end 57.35061 23.664644) (width 1.2) (layer F.Cu) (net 1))
 (segment (start 57.35061 23.664644) (end 53.015254 28) (width 1.2) (layer F.Cu) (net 1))
 (segment (start 53.015254 28) (end 51 28) (width 1.2) (layer F.Cu) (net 1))
 (segment (start 46.629289 21.64939) (end 46.664644 21.64939) (width 1.2) (layer F.Cu) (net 1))
 (segment (start 46.664644 21.64939) (end 51 25.984746) (width 1.2) (layer F.Cu) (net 1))
 (segment (start 51 25.984746) (end 51 28) (width 1.2) (layer F.Cu) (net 1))
 (segment (start 55.370711 21.64939) (end 55.335356 21.64939) (width 1.2) (layer F.Cu) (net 1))
 (segment (start 55.335356 21.64939) (end 51 25.984746) (width 1.2) (layer F.Cu) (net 1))
 (segment (start 51 25.984746) (end 51 28) (width 1.2) (layer F.Cu) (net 1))
 (segment (start 44.37439 23.90061) (end 42.575 25.7) (width 1.2) (layer B.Cu) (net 1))
 (segment (start 42.575 25.7) (end 42.575 26.725) (width 1.2) (layer B.Cu) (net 1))
 (segment (start 44.34939 32.07439) (end 42.6 30.325) (width 1.2) (layer B.Cu) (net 1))
 (segment (start 42.6 30.325) (end 42.6 29.5) (width 1.2) (layer B.Cu) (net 1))
 (segment (start 51 28) (end 51 30.12132) (width 2) (layer F.Cu) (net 1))
 (segment (start 51 28) (end 48.87868 28) (width 2) (layer F.Cu) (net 1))
 (segment (start 51 28) (end 53.12132 28) (width 2) (layer F.Cu) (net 1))
 (segment (start 51 28) (end 51 25.87868) (width 2) (layer F.Cu) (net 1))
 (segment (start 53.1 28) (end 53.12132 28) (width 1) (layer F.Cu) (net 1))
 (segment (start 51 28) (end 53.1 28) (width 1) (layer F.Cu) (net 1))
 (segment (start 28 56) (end 28 63) (width 2) (layer F.Cu) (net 1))
 (segment (start 28 56) (end 21 56) (width 2) (layer F.Cu) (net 1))
 (segment (start 28 56) (end 28 49) (width 2) (layer F.Cu) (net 1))
 (segment (start 28 56) (end 35 56) (width 2) (layer F.Cu) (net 1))
 (segment (start 52.8 29.8) (end 51 28) (width 0.8) (layer B.Cu) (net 2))
 (segment (start 49.2 29.8) (end 51 28) (width 0.8) (layer B.Cu) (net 2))
 (segment (start 49.2 26.2) (end 51 28) (width 0.8) (layer B.Cu) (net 2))
 (segment (start 52.8 26.2) (end 51 28) (width 0.8) (layer B.Cu) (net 2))
 (segment (start 51 28) (end 54.8 28) (width 0.8) (layer B.Cu) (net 2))
 (segment (start 54.8 28) (end 57.5 25.3) (width 0.8) (layer B.Cu) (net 2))
 (segment (start 58.75 25.3) (end 59.425 25.975) (width 0.8) (layer B.Cu) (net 2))
 (segment (start 57.5 25.3) (end 58.75 25.3) (width 0.8) (layer B.Cu) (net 2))
 (segment (start 59.425 25.975) (end 59.425 26.75) (width 0.8) (layer B.Cu) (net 2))
 (segment (start 54.8 28) (end 57.425 30.625) (width 0.8) (layer B.Cu) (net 2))
 (segment (start 58.8 30.625) (end 59.425 30) (width 0.8) (layer B.Cu) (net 2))
 (segment (start 57.425 30.625) (end 58.8 30.625) (width 0.8) (layer B.Cu) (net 2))
 (segment (start 59.425 30) (end 59.425 29.25) (width 0.8) (layer B.Cu) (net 2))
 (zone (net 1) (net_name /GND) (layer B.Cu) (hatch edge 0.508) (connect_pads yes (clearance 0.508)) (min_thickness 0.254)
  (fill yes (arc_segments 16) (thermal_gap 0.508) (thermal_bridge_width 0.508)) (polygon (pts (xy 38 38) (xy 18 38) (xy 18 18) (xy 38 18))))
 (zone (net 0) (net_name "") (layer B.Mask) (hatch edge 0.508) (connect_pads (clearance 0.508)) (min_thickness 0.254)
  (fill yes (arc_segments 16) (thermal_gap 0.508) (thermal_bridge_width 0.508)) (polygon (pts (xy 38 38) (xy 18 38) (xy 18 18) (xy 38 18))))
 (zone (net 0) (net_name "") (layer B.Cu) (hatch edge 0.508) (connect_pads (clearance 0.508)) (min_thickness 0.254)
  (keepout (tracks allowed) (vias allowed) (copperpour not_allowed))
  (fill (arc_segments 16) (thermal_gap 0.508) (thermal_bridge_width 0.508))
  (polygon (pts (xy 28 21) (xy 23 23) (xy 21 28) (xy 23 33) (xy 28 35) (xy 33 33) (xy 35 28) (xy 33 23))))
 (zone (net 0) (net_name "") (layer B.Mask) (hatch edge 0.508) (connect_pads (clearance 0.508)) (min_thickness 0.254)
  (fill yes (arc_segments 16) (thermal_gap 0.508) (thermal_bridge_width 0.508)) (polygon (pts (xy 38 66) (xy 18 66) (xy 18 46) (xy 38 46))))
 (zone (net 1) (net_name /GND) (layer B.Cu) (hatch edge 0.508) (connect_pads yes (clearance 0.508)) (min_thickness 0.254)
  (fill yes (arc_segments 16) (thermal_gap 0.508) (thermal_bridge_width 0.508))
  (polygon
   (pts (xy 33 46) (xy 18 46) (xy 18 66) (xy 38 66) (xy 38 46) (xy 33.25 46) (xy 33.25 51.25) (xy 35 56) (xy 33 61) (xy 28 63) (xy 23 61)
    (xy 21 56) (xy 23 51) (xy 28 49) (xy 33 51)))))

